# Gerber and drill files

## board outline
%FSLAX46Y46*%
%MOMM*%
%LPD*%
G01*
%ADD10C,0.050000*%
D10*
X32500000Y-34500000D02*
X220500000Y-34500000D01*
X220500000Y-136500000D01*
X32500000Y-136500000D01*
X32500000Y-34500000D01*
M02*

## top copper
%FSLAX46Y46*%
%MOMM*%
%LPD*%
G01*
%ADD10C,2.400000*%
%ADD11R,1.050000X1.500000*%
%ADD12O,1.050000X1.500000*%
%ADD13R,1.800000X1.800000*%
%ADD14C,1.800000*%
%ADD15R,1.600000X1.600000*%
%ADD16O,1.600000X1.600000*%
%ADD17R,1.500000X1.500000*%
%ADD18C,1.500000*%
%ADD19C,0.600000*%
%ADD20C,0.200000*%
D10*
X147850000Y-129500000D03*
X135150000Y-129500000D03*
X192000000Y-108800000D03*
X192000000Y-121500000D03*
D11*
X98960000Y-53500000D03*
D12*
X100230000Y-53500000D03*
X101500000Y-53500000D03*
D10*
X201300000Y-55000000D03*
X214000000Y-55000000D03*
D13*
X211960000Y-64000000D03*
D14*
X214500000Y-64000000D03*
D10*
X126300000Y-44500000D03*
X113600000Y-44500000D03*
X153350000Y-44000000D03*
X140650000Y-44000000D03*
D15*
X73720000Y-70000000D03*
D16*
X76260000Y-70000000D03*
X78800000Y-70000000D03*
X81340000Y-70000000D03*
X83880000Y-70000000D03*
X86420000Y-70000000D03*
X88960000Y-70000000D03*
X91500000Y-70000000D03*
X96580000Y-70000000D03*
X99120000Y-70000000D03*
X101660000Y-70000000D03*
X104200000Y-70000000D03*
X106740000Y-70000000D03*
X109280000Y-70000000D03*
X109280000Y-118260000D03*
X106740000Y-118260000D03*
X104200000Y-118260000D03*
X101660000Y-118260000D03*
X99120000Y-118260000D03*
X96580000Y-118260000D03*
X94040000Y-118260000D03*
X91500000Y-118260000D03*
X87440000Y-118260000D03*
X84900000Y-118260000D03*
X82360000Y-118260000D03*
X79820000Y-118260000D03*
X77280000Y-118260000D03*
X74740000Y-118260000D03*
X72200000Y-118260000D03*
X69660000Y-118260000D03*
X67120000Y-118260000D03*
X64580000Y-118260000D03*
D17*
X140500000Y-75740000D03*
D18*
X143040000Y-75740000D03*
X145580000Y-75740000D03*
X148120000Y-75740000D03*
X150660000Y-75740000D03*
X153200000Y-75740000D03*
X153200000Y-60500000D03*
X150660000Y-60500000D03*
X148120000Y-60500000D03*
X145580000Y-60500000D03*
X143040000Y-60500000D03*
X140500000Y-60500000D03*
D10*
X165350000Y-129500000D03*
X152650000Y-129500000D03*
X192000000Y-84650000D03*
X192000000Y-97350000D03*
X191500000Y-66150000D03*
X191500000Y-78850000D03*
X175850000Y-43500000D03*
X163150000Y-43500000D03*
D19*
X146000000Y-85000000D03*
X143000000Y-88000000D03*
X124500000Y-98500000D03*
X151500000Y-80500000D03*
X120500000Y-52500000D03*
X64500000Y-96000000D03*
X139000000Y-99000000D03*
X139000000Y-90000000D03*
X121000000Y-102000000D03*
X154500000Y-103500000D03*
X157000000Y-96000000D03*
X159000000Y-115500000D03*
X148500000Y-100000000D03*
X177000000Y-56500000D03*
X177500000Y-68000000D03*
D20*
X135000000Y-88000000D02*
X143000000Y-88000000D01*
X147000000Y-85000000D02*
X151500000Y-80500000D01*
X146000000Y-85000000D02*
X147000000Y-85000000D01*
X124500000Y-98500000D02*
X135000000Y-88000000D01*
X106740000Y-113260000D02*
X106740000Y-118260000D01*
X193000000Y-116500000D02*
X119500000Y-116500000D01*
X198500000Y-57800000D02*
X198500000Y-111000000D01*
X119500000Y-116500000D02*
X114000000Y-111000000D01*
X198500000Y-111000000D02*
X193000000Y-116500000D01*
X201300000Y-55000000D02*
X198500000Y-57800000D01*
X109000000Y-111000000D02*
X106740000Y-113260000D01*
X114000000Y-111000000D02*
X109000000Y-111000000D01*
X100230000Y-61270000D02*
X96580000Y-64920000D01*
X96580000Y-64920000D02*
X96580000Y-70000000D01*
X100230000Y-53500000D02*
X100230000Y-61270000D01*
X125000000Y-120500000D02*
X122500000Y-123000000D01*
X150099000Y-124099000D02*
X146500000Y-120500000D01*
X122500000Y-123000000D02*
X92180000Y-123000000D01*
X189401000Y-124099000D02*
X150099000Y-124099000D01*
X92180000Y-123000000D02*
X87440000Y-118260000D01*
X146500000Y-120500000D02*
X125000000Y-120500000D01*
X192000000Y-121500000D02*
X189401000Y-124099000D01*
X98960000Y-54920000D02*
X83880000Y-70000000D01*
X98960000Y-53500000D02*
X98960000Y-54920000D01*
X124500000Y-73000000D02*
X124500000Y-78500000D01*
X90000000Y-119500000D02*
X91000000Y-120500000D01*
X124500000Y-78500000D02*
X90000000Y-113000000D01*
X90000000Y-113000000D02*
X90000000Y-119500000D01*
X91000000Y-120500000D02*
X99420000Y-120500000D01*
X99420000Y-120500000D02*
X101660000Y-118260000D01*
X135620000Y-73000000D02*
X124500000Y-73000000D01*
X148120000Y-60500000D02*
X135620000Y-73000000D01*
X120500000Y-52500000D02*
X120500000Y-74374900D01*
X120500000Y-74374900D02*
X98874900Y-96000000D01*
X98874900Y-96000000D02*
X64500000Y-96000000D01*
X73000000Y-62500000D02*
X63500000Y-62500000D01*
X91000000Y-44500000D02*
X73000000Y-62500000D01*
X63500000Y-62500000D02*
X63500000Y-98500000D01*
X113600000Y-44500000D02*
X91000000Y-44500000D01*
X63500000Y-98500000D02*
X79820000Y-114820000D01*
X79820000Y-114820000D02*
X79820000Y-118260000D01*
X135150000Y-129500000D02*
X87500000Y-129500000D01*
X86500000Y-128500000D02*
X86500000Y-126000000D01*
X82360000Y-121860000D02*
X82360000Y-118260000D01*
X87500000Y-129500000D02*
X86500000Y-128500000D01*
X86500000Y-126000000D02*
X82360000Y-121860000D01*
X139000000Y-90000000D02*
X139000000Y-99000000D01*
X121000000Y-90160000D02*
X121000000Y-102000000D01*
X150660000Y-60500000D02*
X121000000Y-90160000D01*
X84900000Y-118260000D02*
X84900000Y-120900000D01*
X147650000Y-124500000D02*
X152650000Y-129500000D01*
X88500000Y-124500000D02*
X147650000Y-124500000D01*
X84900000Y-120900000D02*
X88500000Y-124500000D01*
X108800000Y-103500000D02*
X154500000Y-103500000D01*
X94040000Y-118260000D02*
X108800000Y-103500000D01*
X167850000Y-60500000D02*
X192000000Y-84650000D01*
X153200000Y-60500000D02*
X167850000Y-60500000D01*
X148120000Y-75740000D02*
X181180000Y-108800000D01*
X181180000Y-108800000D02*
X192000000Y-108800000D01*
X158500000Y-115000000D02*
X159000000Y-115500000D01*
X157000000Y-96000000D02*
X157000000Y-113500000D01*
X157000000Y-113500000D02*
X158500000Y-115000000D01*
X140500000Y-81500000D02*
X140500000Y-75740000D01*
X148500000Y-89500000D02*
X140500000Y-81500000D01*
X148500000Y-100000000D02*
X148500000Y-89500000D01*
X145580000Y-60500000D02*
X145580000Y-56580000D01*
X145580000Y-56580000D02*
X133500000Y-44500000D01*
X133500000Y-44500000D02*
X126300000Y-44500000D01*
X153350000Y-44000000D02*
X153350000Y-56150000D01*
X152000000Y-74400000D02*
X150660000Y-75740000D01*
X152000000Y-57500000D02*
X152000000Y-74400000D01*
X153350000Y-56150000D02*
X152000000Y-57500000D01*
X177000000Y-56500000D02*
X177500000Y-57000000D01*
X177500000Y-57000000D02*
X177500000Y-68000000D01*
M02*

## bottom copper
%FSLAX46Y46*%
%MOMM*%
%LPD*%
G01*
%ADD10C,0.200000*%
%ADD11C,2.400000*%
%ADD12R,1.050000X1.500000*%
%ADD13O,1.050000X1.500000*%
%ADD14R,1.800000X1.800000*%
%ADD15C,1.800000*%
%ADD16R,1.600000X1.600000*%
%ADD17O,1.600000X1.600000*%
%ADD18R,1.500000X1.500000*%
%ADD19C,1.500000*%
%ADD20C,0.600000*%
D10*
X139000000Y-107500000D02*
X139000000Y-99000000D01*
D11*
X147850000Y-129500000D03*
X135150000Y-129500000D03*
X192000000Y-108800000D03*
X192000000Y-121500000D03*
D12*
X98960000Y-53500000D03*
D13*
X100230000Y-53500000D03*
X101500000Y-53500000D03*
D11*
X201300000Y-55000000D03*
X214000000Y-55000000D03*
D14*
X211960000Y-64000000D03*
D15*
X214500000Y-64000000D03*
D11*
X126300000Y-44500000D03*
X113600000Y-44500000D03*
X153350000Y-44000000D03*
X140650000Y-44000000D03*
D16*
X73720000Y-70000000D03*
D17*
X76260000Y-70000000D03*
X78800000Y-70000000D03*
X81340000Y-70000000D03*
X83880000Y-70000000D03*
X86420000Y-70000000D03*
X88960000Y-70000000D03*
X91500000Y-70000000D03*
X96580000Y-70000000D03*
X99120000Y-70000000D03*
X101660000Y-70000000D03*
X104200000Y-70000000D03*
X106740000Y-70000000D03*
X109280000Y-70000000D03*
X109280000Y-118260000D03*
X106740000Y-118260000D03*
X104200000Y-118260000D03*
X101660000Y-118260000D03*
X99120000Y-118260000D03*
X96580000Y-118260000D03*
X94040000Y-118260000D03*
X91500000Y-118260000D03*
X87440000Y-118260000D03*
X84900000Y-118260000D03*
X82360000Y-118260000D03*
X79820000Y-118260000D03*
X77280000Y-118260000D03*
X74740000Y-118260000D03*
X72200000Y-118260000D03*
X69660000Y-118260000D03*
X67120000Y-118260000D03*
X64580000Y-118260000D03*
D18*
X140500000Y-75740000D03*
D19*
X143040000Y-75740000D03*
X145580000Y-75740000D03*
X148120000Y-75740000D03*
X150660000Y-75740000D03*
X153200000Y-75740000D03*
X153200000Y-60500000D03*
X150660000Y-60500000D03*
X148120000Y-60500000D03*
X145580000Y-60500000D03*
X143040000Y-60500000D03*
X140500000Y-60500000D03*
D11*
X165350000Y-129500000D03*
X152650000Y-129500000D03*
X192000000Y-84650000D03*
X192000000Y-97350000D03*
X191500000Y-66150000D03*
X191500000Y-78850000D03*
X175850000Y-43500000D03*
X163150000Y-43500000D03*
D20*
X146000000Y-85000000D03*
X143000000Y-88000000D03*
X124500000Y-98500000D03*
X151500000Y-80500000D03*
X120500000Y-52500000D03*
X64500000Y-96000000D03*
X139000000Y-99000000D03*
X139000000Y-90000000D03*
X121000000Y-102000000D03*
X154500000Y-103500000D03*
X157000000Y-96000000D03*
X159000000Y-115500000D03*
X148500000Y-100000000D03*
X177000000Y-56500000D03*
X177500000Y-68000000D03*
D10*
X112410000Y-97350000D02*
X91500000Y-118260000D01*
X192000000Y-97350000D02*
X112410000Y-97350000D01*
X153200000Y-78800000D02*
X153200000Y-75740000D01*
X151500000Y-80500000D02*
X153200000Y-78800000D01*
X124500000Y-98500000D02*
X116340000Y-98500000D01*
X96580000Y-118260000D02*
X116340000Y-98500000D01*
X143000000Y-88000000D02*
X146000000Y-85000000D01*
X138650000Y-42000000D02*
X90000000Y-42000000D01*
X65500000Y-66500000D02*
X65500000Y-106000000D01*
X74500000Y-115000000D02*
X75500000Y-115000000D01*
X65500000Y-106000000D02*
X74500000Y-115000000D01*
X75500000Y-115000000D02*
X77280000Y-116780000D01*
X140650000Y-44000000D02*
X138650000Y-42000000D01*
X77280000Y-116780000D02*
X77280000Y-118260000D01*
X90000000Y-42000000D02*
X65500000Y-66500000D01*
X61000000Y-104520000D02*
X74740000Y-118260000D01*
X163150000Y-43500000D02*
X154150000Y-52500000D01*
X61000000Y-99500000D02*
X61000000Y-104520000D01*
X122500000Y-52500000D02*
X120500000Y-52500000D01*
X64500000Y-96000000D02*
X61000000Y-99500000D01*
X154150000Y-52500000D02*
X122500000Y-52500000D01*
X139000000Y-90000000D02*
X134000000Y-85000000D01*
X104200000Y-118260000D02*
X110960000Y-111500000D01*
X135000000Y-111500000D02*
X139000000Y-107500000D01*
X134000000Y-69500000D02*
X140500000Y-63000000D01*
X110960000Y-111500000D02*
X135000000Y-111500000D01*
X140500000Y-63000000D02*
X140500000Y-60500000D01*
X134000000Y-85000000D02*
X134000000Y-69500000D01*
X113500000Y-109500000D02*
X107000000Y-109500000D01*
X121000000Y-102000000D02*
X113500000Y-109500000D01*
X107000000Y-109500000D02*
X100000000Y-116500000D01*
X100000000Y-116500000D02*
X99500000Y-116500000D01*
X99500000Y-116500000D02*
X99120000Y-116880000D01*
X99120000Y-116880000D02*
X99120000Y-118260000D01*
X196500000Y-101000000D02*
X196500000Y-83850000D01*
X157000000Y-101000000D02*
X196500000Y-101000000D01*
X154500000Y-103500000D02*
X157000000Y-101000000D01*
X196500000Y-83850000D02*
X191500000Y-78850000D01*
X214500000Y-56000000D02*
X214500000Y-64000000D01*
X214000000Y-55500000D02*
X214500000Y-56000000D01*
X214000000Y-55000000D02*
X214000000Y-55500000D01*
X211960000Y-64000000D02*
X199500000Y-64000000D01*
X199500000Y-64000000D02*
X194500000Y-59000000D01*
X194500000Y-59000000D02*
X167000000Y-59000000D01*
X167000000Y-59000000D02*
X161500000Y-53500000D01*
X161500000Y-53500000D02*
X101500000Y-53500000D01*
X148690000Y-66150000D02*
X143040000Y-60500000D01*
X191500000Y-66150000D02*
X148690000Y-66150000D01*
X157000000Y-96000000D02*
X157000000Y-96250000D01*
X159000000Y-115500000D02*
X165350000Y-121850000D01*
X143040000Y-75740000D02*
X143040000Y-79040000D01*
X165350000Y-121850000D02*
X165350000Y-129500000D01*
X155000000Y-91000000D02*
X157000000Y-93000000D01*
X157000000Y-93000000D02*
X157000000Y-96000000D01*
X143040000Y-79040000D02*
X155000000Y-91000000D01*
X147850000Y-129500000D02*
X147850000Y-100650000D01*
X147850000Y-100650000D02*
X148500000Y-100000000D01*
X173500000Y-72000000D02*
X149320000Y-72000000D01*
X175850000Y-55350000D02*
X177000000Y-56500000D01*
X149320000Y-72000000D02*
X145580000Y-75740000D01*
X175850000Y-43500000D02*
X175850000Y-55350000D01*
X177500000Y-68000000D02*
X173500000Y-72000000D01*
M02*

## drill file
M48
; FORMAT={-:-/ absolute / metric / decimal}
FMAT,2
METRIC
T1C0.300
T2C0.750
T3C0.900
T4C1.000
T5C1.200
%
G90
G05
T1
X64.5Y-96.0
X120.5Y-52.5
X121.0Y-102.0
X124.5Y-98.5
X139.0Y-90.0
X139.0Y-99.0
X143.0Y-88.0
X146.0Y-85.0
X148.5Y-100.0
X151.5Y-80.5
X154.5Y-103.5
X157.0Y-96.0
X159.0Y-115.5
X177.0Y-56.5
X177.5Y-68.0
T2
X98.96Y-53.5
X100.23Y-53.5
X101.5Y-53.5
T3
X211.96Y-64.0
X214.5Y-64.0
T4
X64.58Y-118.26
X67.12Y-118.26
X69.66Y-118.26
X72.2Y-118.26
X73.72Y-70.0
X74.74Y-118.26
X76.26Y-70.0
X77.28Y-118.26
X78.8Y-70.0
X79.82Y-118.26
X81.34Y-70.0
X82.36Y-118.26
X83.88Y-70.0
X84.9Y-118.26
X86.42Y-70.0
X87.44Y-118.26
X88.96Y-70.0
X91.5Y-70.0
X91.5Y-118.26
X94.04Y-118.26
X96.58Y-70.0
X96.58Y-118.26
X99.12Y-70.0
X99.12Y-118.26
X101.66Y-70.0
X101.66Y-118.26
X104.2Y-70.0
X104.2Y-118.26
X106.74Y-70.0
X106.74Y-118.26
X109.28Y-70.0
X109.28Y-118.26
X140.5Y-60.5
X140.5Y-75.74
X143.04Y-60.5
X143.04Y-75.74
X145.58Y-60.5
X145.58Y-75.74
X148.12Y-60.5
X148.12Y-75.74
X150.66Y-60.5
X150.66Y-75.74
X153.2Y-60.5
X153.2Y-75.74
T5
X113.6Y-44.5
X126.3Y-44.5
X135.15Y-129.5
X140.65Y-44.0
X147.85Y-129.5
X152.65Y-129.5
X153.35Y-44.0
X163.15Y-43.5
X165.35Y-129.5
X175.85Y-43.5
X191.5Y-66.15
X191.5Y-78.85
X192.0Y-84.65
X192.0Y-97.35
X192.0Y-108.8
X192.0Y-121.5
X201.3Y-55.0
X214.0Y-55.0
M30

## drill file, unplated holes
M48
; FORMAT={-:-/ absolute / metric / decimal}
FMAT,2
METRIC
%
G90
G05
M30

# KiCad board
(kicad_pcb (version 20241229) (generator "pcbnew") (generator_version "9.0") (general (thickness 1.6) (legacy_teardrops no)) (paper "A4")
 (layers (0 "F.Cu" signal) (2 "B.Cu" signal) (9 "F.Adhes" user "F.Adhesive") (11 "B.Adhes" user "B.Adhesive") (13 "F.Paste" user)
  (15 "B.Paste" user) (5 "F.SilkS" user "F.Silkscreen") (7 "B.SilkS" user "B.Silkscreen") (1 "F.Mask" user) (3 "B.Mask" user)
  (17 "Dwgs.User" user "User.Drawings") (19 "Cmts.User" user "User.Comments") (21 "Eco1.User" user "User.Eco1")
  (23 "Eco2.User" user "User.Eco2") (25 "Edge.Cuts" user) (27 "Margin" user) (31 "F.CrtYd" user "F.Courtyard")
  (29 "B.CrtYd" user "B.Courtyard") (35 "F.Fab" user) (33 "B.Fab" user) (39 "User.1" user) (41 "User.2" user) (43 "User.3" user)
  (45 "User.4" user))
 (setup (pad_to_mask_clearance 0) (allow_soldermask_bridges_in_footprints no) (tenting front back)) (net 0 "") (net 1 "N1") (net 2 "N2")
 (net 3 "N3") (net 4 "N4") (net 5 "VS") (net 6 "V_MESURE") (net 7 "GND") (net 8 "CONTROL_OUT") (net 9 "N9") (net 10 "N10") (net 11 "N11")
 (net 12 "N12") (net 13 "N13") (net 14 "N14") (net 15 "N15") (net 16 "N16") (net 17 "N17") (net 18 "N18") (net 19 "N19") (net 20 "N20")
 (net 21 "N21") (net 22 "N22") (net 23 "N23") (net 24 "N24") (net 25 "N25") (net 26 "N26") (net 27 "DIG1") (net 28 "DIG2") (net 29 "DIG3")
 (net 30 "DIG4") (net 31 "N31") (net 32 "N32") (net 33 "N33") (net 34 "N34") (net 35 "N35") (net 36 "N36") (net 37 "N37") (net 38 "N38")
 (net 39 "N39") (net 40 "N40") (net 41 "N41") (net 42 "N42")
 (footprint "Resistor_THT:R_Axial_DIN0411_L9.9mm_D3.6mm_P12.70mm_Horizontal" (layer "F.Cu") (at 147.85 129.5 180)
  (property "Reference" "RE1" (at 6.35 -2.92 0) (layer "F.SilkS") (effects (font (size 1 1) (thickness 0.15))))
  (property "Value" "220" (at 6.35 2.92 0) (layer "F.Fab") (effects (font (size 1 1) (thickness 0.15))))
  (pad "1" thru_hole circle (at 0 0 180) (size 2.4 2.4) (drill 1.2) (layers "*.Cu" "*.Mask") (remove_unused_layers no) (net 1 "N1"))
  (pad "2" thru_hole circle (at 12.7 0 180) (size 2.4 2.4) (drill 1.2) (layers "*.Cu" "*.Mask") (remove_unused_layers no) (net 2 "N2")))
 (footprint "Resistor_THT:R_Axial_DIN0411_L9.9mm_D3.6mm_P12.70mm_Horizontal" (layer "F.Cu") (at 192 108.8 -90)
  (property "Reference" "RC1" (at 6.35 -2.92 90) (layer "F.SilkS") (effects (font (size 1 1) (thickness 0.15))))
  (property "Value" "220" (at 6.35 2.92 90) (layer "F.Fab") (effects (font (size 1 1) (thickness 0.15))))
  (pad "1" thru_hole circle (at 0 0 270) (size 2.4 2.4) (drill 1.2) (layers "*.Cu" "*.Mask") (remove_unused_layers no) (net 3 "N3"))
  (pad "2" thru_hole circle (at 12.7 0 270) (size 2.4 2.4) (drill 1.2) (layers "*.Cu" "*.Mask") (remove_unused_layers no) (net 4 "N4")))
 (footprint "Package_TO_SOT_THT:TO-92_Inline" (layer "F.Cu") (at 98.96 53.5)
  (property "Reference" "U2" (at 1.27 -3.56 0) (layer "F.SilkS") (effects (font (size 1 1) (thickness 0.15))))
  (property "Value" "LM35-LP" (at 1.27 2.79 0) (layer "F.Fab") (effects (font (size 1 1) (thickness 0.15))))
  (pad "1" thru_hole rect (at 0 0) (size 1.05 1.5) (drill 0.75) (layers "*.Cu" "*.Mask") (remove_unused_layers no) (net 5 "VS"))
  (pad "2" thru_hole oval (at 1.27 0) (size 1.05 1.5) (drill 0.75) (layers "*.Cu" "*.Mask") (remove_unused_layers no) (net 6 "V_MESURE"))
  (pad "3" thru_hole oval (at 2.54 0) (size 1.05 1.5) (drill 0.75) (layers "*.Cu" "*.Mask") (remove_unused_layers no) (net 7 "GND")))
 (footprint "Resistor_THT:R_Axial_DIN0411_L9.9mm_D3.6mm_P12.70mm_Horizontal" (layer "F.Cu") (at 201.3 55)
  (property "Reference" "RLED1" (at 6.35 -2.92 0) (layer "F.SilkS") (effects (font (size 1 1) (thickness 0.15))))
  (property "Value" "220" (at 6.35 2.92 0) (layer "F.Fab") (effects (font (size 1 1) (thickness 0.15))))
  (pad "1" thru_hole circle (at 0 0) (size 2.4 2.4) (drill 1.2) (layers "*.Cu" "*.Mask") (remove_unused_layers no) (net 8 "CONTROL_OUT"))
  (pad "2" thru_hole circle (at 12.7 0) (size 2.4 2.4) (drill 1.2) (layers "*.Cu" "*.Mask") (remove_unused_layers no) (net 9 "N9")))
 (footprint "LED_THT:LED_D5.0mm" (layer "F.Cu") (at 211.96 64)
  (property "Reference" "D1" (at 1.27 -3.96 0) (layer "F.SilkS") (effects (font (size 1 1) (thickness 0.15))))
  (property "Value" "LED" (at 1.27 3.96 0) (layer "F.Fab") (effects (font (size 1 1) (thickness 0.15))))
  (pad "1" thru_hole rect (at 0 0) (size 1.8 1.8) (drill 0.9) (layers "*.Cu" "*.Mask") (remove_unused_layers no) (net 7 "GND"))
  (pad "2" thru_hole circle (at 2.54 0) (size 1.8 1.8) (drill 0.9) (layers "*.Cu" "*.Mask") (remove_unused_layers no) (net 9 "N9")))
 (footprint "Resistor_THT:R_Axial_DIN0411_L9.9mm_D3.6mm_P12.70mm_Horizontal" (layer "F.Cu") (at 126.3 44.5 180)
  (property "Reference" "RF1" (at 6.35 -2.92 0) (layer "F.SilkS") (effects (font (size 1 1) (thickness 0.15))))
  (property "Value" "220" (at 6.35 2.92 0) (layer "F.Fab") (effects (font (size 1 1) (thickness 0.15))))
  (pad "1" thru_hole circle (at 0 0 180) (size 2.4 2.4) (drill 1.2) (layers "*.Cu" "*.Mask") (remove_unused_layers no) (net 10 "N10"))
  (pad "2" thru_hole circle (at 12.7 0 180) (size 2.4 2.4) (drill 1.2) (layers "*.Cu" "*.Mask") (remove_unused_layers no) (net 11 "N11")))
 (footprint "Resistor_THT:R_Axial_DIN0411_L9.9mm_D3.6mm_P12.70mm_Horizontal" (layer "F.Cu") (at 153.35 44 180)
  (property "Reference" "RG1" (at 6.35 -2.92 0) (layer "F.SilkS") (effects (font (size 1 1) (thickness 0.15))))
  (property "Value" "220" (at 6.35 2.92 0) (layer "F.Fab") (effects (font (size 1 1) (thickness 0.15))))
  (pad "1" thru_hole circle (at 0 0 180) (size 2.4 2.4) (drill 1.2) (layers "*.Cu" "*.Mask") (remove_unused_layers no) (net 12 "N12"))
  (pad "2" thru_hole circle (at 12.7 0 180) (size 2.4 2.4) (drill 1.2) (layers "*.Cu" "*.Mask") (remove_unused_layers no) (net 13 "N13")))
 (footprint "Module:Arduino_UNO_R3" (layer "F.Cu") (at 73.72 70)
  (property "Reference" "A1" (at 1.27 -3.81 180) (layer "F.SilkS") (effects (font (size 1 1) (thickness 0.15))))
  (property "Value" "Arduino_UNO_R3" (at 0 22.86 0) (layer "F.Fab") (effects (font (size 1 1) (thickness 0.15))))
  (pad "1" thru_hole rect (at 0 0 90) (size 1.6 1.6) (drill 1) (layers "*.Cu" "*.Mask") (remove_unused_layers no) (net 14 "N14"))
  (pad "2" thru_hole oval (at 2.54 0 90) (size 1.6 1.6) (drill 1) (layers "*.Cu" "*.Mask") (remove_unused_layers no) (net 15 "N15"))
  (pad "3" thru_hole oval (at 5.08 0 90) (size 1.6 1.6) (drill 1) (layers "*.Cu" "*.Mask") (remove_unused_layers no) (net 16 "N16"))
  (pad "4" thru_hole oval (at 7.62 0 90) (size 1.6 1.6) (drill 1) (layers "*.Cu" "*.Mask") (remove_unused_layers no) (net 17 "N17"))
  (pad "5" thru_hole oval (at 10.16 0 90) (size 1.6 1.6) (drill 1) (layers "*.Cu" "*.Mask") (remove_unused_layers no) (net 5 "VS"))
  (pad "6" thru_hole oval (at 12.7 0 90) (size 1.6 1.6) (drill 1) (layers "*.Cu" "*.Mask") (remove_unused_layers no) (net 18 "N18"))
  (pad "7" thru_hole oval (at 15.24 0 90) (size 1.6 1.6) (drill 1) (layers "*.Cu" "*.Mask") (remove_unused_layers no) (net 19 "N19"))
  (pad "8" thru_hole oval (at 17.78 0 90) (size 1.6 1.6) (drill 1) (layers "*.Cu" "*.Mask") (remove_unused_layers no) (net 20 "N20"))
  (pad "9" thru_hole oval (at 22.86 0 90) (size 1.6 1.6) (drill 1) (layers "*.Cu" "*.Mask") (remove_unused_layers no) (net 6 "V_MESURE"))
  (pad "10" thru_hole oval (at 25.4 0 90) (size 1.6 1.6) (drill 1) (layers "*.Cu" "*.Mask") (remove_unused_layers no) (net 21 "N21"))
  (pad "11" thru_hole oval (at 27.94 0 90) (size 1.6 1.6) (drill 1) (layers "*.Cu" "*.Mask") (remove_unused_layers no) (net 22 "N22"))
  (pad "12" thru_hole oval (at 30.48 0 90) (size 1.6 1.6) (drill 1) (layers "*.Cu" "*.Mask") (remove_unused_layers no) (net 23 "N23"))
  (pad "13" thru_hole oval (at 33.02 0 90) (size 1.6 1.6) (drill 1) (layers "*.Cu" "*.Mask") (remove_unused_layers no) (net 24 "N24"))
  (pad "14" thru_hole oval (at 35.56 0 90) (size 1.6 1.6) (drill 1) (layers "*.Cu" "*.Mask") (remove_unused_layers no) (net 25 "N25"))
  (pad "15" thru_hole oval (at 35.56 48.26 90) (size 1.6 1.6) (drill 1) (layers "*.Cu" "*.Mask") (remove_unused_layers no) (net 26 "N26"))
  (pad "16" thru_hole oval (at 33.02 48.26 90) (size 1.6 1.6) (drill 1) (layers "*.Cu" "*.Mask") (remove_unused_layers no)
   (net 8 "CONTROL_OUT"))
  (pad "17" thru_hole oval (at 30.48 48.26 90) (size 1.6 1.6) (drill 1) (layers "*.Cu" "*.Mask") (remove_unused_layers no) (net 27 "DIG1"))
  (pad "18" thru_hole oval (at 27.94 48.26 90) (size 1.6 1.6) (drill 1) (layers "*.Cu" "*.Mask") (remove_unused_layers no) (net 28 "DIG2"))
  (pad "19" thru_hole oval (at 25.4 48.26 90) (size 1.6 1.6) (drill 1) (layers "*.Cu" "*.Mask") (remove_unused_layers no) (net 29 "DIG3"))
  (pad "20" thru_hole oval (at 22.86 48.26 90) (size 1.6 1.6) (drill 1) (layers "*.Cu" "*.Mask") (remove_unused_layers no) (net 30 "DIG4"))
  (pad "21" thru_hole oval (at 20.32 48.26 90) (size 1.6 1.6) (drill 1) (layers "*.Cu" "*.Mask") (remove_unused_layers no) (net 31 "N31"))
  (pad "22" thru_hole oval (at 17.78 48.26 90) (size 1.6 1.6) (drill 1) (layers "*.Cu" "*.Mask") (remove_unused_layers no) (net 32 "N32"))
  (pad "23" thru_hole oval (at 13.72 48.26 90) (size 1.6 1.6) (drill 1) (layers "*.Cu" "*.Mask") (remove_unused_layers no) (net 4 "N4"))
  (pad "24" thru_hole oval (at 11.18 48.26 90) (size 1.6 1.6) (drill 1) (layers "*.Cu" "*.Mask") (remove_unused_layers no) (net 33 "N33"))
  (pad "25" thru_hole oval (at 8.64 48.26 90) (size 1.6 1.6) (drill 1) (layers "*.Cu" "*.Mask") (remove_unused_layers no) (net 2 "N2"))
  (pad "26" thru_hole oval (at 6.1 48.26 90) (size 1.6 1.6) (drill 1) (layers "*.Cu" "*.Mask") (remove_unused_layers no) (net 11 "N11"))
  (pad "27" thru_hole oval (at 3.56 48.26 90) (size 1.6 1.6) (drill 1) (layers "*.Cu" "*.Mask") (remove_unused_layers no) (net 13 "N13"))
  (pad "28" thru_hole oval (at 1.02 48.26 90) (size 1.6 1.6) (drill 1) (layers "*.Cu" "*.Mask") (remove_unused_layers no) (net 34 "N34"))
  (pad "29" thru_hole oval (at -1.52 48.26 90) (size 1.6 1.6) (drill 1) (layers "*.Cu" "*.Mask") (remove_unused_layers no) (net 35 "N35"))
  (pad "30" thru_hole oval (at -4.06 48.26 90) (size 1.6 1.6) (drill 1) (layers "*.Cu" "*.Mask") (remove_unused_layers no) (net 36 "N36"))
  (pad "31" thru_hole oval (at -6.6 48.26 90) (size 1.6 1.6) (drill 1) (layers "*.Cu" "*.Mask") (remove_unused_layers no) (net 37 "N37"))
  (pad "32" thru_hole oval (at -9.14 48.26 90) (size 1.6 1.6) (drill 1) (layers "*.Cu" "*.Mask") (remove_unused_layers no) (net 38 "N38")))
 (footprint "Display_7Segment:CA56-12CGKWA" (layer "F.Cu") (at 140.5 75.74 90)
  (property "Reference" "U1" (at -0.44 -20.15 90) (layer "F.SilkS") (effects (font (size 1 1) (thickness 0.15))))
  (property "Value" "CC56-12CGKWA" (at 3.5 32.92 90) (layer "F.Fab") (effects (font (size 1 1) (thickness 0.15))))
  (pad "1" thru_hole rect (at 0 0 90) (size 1.5 1.5) (drill 1) (layers "*.Cu" "*.Mask") (remove_unused_layers no) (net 1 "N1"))
  (pad "2" thru_hole circle (at 0 2.54 90) (size 1.5 1.5) (drill 1) (layers "*.Cu" "*.Mask") (remove_unused_layers no) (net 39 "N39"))
  (pad "3" thru_hole circle (at 0 5.08 90) (size 1.5 1.5) (drill 1) (layers "*.Cu" "*.Mask") (remove_unused_layers no) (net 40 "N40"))
  (pad "4" thru_hole circle (at 0 7.62 90) (size 1.5 1.5) (drill 1) (layers "*.Cu" "*.Mask") (remove_unused_layers no) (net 3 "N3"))
  (pad "5" thru_hole circle (at 0 10.16 90) (size 1.5 1.5) (drill 1) (layers "*.Cu" "*.Mask") (remove_unused_layers no) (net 12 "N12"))
  (pad "6" thru_hole circle (at 0 12.7 90) (size 1.5 1.5) (drill 1) (layers "*.Cu" "*.Mask") (remove_unused_layers no) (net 30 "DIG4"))
  (pad "7" thru_hole circle (at 15.24 12.7 90) (size 1.5 1.5) (drill 1) (layers "*.Cu" "*.Mask") (remove_unused_layers no) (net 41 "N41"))
  (pad "8" thru_hole circle (at 15.24 10.16 90) (size 1.5 1.5) (drill 1) (layers "*.Cu" "*.Mask") (remove_unused_layers no) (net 29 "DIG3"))
  (pad "9" thru_hole circle (at 15.24 7.62 90) (size 1.5 1.5) (drill 1) (layers "*.Cu" "*.Mask") (remove_unused_layers no) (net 28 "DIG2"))
  (pad "10" thru_hole circle (at 15.24 5.08 90) (size 1.5 1.5) (drill 1) (layers "*.Cu" "*.Mask") (remove_unused_layers no) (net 10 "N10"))
  (pad "11" thru_hole circle (at 15.24 2.54 90) (size 1.5 1.5) (drill 1) (layers "*.Cu" "*.Mask") (remove_unused_layers no) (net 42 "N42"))
  (pad "12" thru_hole circle (at 15.24 0 90) (size 1.5 1.5) (drill 1) (layers "*.Cu" "*.Mask") (remove_unused_layers no) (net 27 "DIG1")))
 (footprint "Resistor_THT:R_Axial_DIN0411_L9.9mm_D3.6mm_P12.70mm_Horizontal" (layer "F.Cu") (at 165.35 129.5 180)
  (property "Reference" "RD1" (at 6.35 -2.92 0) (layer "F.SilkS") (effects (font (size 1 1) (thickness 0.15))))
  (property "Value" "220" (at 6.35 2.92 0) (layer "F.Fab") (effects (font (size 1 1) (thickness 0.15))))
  (pad "1" thru_hole circle (at 0 0 180) (size 2.4 2.4) (drill 1.2) (layers "*.Cu" "*.Mask") (remove_unused_layers no) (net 39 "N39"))
  (pad "2" thru_hole circle (at 12.7 0 180) (size 2.4 2.4) (drill 1.2) (layers "*.Cu" "*.Mask") (remove_unused_layers no) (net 33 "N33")))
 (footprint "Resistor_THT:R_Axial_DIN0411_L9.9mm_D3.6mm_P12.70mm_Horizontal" (layer "F.Cu") (at 192 84.65 -90)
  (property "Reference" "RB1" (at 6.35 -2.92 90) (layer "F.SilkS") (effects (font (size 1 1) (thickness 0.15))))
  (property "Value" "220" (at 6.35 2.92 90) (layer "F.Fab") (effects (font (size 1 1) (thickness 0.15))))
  (pad "1" thru_hole circle (at 0 0 270) (size 2.4 2.4) (drill 1.2) (layers "*.Cu" "*.Mask") (remove_unused_layers no) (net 41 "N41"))
  (pad "2" thru_hole circle (at 12.7 0 270) (size 2.4 2.4) (drill 1.2) (layers "*.Cu" "*.Mask") (remove_unused_layers no) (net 32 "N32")))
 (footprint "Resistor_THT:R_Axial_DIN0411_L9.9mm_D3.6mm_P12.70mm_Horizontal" (layer "F.Cu") (at 191.5 66.15 -90)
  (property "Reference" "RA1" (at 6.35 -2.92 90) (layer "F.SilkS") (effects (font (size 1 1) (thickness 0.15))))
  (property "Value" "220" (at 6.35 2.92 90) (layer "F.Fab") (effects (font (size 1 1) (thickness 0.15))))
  (pad "1" thru_hole circle (at 0 0 270) (size 2.4 2.4) (drill 1.2) (layers "*.Cu" "*.Mask") (remove_unused_layers no) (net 42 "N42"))
  (pad "2" thru_hole circle (at 12.7 0 270) (size 2.4 2.4) (drill 1.2) (layers "*.Cu" "*.Mask") (remove_unused_layers no) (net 31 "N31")))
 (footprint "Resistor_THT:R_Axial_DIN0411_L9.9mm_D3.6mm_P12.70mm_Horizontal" (layer "F.Cu") (at 175.85 43.5 180)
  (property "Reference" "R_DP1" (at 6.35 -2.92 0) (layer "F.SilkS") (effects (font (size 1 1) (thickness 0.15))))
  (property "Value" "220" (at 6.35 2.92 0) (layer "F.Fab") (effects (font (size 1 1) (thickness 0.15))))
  (pad "1" thru_hole circle (at 0 0 180) (size 2.4 2.4) (drill 1.2) (layers "*.Cu" "*.Mask") (remove_unused_layers no) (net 40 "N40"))
  (pad "2" thru_hole circle (at 12.7 0 180) (size 2.4 2.4) (drill 1.2) (layers "*.Cu" "*.Mask") (remove_unused_layers no) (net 34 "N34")))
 (gr_line (start 139 107.5) (end 139 99) (stroke (width 0.2) (type default)) (layer "B.Cu") (net 27))
 (gr_rect (start 32.5 34.5) (end 220.5 136.5) (stroke (width 0.05) (type default)) (fill no) (layer "Edge.Cuts"))
 (segment (start 112.41 97.35) (end 91.5 118.26) (width 0.2) (layer "B.Cu") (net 32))
 (segment (start 192 97.35) (end 112.41 97.35) (width 0.2) (layer "B.Cu") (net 32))
 (segment (start 135 88) (end 143 88) (width 0.2) (layer "F.Cu") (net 30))
 (segment (start 147 85) (end 151.5 80.5) (width 0.2) (layer "F.Cu") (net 30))
 (segment (start 146 85) (end 147 85) (width 0.2) (layer "F.Cu") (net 30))
 (segment (start 124.5 98.5) (end 135 88) (width 0.2) (layer "F.Cu") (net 30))
 (via (at 146 85) (size 0.6) (drill 0.3) (layers "F.Cu" "B.Cu") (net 30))
 (via (at 143 88) (size 0.6) (drill 0.3) (layers "F.Cu" "B.Cu") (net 30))
 (via (at 124.5 98.5) (size 0.6) (drill 0.3) (layers "F.Cu" "B.Cu") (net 30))
 (via (at 151.5 80.5) (size 0.6) (drill 0.3) (layers "F.Cu" "B.Cu") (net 30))
 (segment (start 153.2 78.8) (end 153.2 75.74) (width 0.2) (layer "B.Cu") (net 30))
 (segment (start 151.5 80.5) (end 153.2 78.8) (width 0.2) (layer "B.Cu") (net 30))
 (segment (start 124.5 98.5) (end 116.34 98.5) (width 0.2) (layer "B.Cu") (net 30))
 (segment (start 96.58 118.26) (end 116.34 98.5) (width 0.2) (layer "B.Cu") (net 30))
 (segment (start 143 88) (end 146 85) (width 0.2) (layer "B.Cu") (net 30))
 (segment (start 106.74 113.26) (end 106.74 118.26) (width 0.2) (layer "F.Cu") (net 8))
 (segment (start 193 116.5) (end 119.5 116.5) (width 0.2) (layer "F.Cu") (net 8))
 (segment (start 198.5 57.8) (end 198.5 111) (width 0.2) (layer "F.Cu") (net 8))
 (segment (start 119.5 116.5) (end 114 111) (width 0.2) (layer "F.Cu") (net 8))
 (segment (start 198.5 111) (end 193 116.5) (width 0.2) (layer "F.Cu") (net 8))
 (segment (start 201.3 55) (end 198.5 57.8) (width 0.2) (layer "F.Cu") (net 8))
 (segment (start 109 111) (end 106.74 113.26) (width 0.2) (layer "F.Cu") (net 8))
 (segment (start 114 111) (end 109 111) (width 0.2) (layer "F.Cu") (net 8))
 (segment (start 138.65 42) (end 90 42) (width 0.2) (layer "B.Cu") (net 13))
 (segment (start 65.5 66.5) (end 65.5 106) (width 0.2) (layer "B.Cu") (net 13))
 (segment (start 74.5 115) (end 75.5 115) (width 0.2) (layer "B.Cu") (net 13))
 (segment (start 65.5 106) (end 74.5 115) (width 0.2) (layer "B.Cu") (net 13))
 (segment (start 75.5 115) (end 77.28 116.78) (width 0.2) (layer "B.Cu") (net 13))
 (segment (start 140.65 44) (end 138.65 42) (width 0.2) (layer "B.Cu") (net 13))
 (segment (start 77.28 116.78) (end 77.28 118.26) (width 0.2) (layer "B.Cu") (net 13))
 (segment (start 90 42) (end 65.5 66.5) (width 0.2) (layer "B.Cu") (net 13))
 (segment (start 100.23 61.27) (end 96.58 64.92) (width 0.2) (layer "F.Cu") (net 6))
 (segment (start 96.58 64.92) (end 96.58 70) (width 0.2) (layer "F.Cu") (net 6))
 (segment (start 100.23 53.5) (end 100.23 61.27) (width 0.2) (layer "F.Cu") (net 6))
 (segment (start 125 120.5) (end 122.5 123) (width 0.2) (layer "F.Cu") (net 4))
 (segment (start 150.099 124.099) (end 146.5 120.5) (width 0.2) (layer "F.Cu") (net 4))
 (segment (start 122.5 123) (end 92.18 123) (width 0.2) (layer "F.Cu") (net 4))
 (segment (start 189.401 124.099) (end 150.099 124.099) (width 0.2) (layer "F.Cu") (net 4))
 (segment (start 92.18 123) (end 87.44 118.26) (width 0.2) (layer "F.Cu") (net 4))
 (segment (start 146.5 120.5) (end 125 120.5) (width 0.2) (layer "F.Cu") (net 4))
 (segment (start 192 121.5) (end 189.401 124.099) (width 0.2) (layer "F.Cu") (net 4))
 (segment (start 98.96 54.92) (end 83.88 70) (width 0.2) (layer "F.Cu") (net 5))
 (segment (start 98.96 53.5) (end 98.96 54.92) (width 0.2) (layer "F.Cu") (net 5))
 (segment (start 124.5 73) (end 124.5 78.5) (width 0.2) (layer "F.Cu") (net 28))
 (segment (start 90 119.5) (end 91 120.5) (width 0.2) (layer "F.Cu") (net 28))
 (segment (start 124.5 78.5) (end 90 113) (width 0.2) (layer "F.Cu") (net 28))
 (segment (start 90 113) (end 90 119.5) (width 0.2) (layer "F.Cu") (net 28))
 (segment (start 91 120.5) (end 99.42 120.5) (width 0.2) (layer "F.Cu") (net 28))
 (segment (start 99.42 120.5) (end 101.66 118.26) (width 0.2) (layer "F.Cu") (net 28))
 (segment (start 135.62 73) (end 124.5 73) (width 0.2) (layer "F.Cu") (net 28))
 (segment (start 148.12 60.5) (end 135.62 73) (width 0.2) (layer "F.Cu") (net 28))
 (segment (start 120.5 52.5) (end 120.5 74.3749) (width 0.2) (layer "F.Cu") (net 34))
 (segment (start 120.5 74.3749) (end 98.8749 96) (width 0.2) (layer "F.Cu") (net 34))
 (segment (start 98.8749 96) (end 64.5 96) (width 0.2) (layer "F.Cu") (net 34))
 (via (at 120.5 52.5) (size 0.6) (drill 0.3) (layers "F.Cu" "B.Cu") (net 34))
 (via (at 64.5 96) (size 0.6) (drill 0.3) (layers "F.Cu" "B.Cu") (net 34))
 (segment (start 61 104.52) (end 74.74 118.26) (width 0.2) (layer "B.Cu") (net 34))
 (segment (start 163.15 43.5) (end 154.15 52.5) (width 0.2) (layer "B.Cu") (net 34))
 (segment (start 61 99.5) (end 61 104.52) (width 0.2) (layer "B.Cu") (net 34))
 (segment (start 122.5 52.5) (end 120.5 52.5) (width 0.2) (layer "B.Cu") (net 34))
 (segment (start 64.5 96) (end 61 99.5) (width 0.2) (layer "B.Cu") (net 34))
 (segment (start 154.15 52.5) (end 122.5 52.5) (width 0.2) (layer "B.Cu") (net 34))
 (segment (start 73 62.5) (end 63.5 62.5) (width 0.2) (layer "F.Cu") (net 11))
 (segment (start 91 44.5) (end 73 62.5) (width 0.2) (layer "F.Cu") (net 11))
 (segment (start 63.5 62.5) (end 63.5 98.5) (width 0.2) (layer "F.Cu") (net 11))
 (segment (start 113.6 44.5) (end 91 44.5) (width 0.2) (layer "F.Cu") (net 11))
 (segment (start 63.5 98.5) (end 79.82 114.82) (width 0.2) (layer "F.Cu") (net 11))
 (segment (start 79.82 114.82) (end 79.82 118.26) (width 0.2) (layer "F.Cu") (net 11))
 (segment (start 135.15 129.5) (end 87.5 129.5) (width 0.2) (layer "F.Cu") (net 2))
 (segment (start 86.5 128.5) (end 86.5 126) (width 0.2) (layer "F.Cu") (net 2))
 (segment (start 82.36 121.86) (end 82.36 118.26) (width 0.2) (layer "F.Cu") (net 2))
 (segment (start 87.5 129.5) (end 86.5 128.5) (width 0.2) (layer "F.Cu") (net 2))
 (segment (start 86.5 126) (end 82.36 121.86) (width 0.2) (layer "F.Cu") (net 2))
 (segment (start 139 90) (end 139 99) (width 0.2) (layer "F.Cu") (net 27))
 (via (at 139 99) (size 0.6) (drill 0.3) (layers "F.Cu" "B.Cu") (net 27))
 (via (at 139 90) (size 0.6) (drill 0.3) (layers "F.Cu" "B.Cu") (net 27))
 (segment (start 139 90) (end 134 85) (width 0.2) (layer "B.Cu") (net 27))
 (segment (start 104.2 118.26) (end 110.96 111.5) (width 0.2) (layer "B.Cu") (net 27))
 (segment (start 135 111.5) (end 139 107.5) (width 0.2) (layer "B.Cu") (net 27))
 (segment (start 134 69.5) (end 140.5 63) (width 0.2) (layer "B.Cu") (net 27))
 (segment (start 110.96 111.5) (end 135 111.5) (width 0.2) (layer "B.Cu") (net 27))
 (segment (start 140.5 63) (end 140.5 60.5) (width 0.2) (layer "B.Cu") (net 27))
 (segment (start 134 85) (end 134 69.5) (width 0.2) (layer "B.Cu") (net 27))
 (segment (start 121 90.16) (end 121 102) (width 0.2) (layer "F.Cu") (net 29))
 (segment (start 150.66 60.5) (end 121 90.16) (width 0.2) (layer "F.Cu") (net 29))
 (via (at 121 102) (size 0.6) (drill 0.3) (layers "F.Cu" "B.Cu") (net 29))
 (segment (start 113.5 109.5) (end 107 109.5) (width 0.2) (layer "B.Cu") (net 29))
 (segment (start 121 102) (end 113.5 109.5) (width 0.2) (layer "B.Cu") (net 29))
 (segment (start 107 109.5) (end 100 116.5) (width 0.2) (layer "B.Cu") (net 29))
 (segment (start 100 116.5) (end 99.5 116.5) (width 0.2) (layer "B.Cu") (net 29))
 (segment (start 99.5 116.5) (end 99.12 116.88) (width 0.2) (layer "B.Cu") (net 29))
 (segment (start 99.12 116.88) (end 99.12 118.26) (width 0.2) (layer "B.Cu") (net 29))
 (segment (start 84.9 118.26) (end 84.9 120.9) (width 0.2) (layer "F.Cu") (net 33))
 (segment (start 147.65 124.5) (end 152.65 129.5) (width 0.2) (layer "F.Cu") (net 33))
 (segment (start 88.5 124.5) (end 147.65 124.5) (width 0.2) (layer "F.Cu") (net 33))
 (segment (start 84.9 120.9) (end 88.5 124.5) (width 0.2) (layer "F.Cu") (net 33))
 (segment (start 108.8 103.5) (end 154.5 103.5) (width 0.2) (layer "F.Cu") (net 31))
 (segment (start 94.04 118.26) (end 108.8 103.5) (width 0.2) (layer "F.Cu") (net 31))
 (via (at 154.5 103.5) (size 0.6) (drill 0.3) (layers "F.Cu" "B.Cu") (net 31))
 (segment (start 196.5 101) (end 196.5 83.85) (width 0.2) (layer "B.Cu") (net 31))
 (segment (start 157 101) (end 196.5 101) (width 0.2) (layer "B.Cu") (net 31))
 (segment (start 154.5 103.5) (end 157 101) (width 0.2) (layer "B.Cu") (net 31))
 (segment (start 196.5 83.85) (end 191.5 78.85) (width 0.2) (layer "B.Cu") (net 31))
 (segment (start 214.5 56) (end 214.5 64) (width 0.2) (layer "B.Cu") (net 9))
 (segment (start 214 55.5) (end 214.5 56) (width 0.2) (layer "B.Cu") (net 9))
 (segment (start 214 55) (end 214 55.5) (width 0.2) (layer "B.Cu") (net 9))
 (segment (start 211.96 64) (end 199.5 64) (width 0.2) (layer "B.Cu") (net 7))
 (segment (start 199.5 64) (end 194.5 59) (width 0.2) (layer "B.Cu") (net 7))
 (segment (start 194.5 59) (end 167 59) (width 0.2) (layer "B.Cu") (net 7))
 (segment (start 167 59) (end 161.5 53.5) (width 0.2) (layer "B.Cu") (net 7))
 (segment (start 161.5 53.5) (end 101.5 53.5) (width 0.2) (layer "B.Cu") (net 7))
 (segment (start 148.69 66.15) (end 143.04 60.5) (width 0.2) (layer "B.Cu") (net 42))
 (segment (start 191.5 66.15) (end 148.69 66.15) (width 0.2) (layer "B.Cu") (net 42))
 (segment (start 167.85 60.5) (end 192 84.65) (width 0.2) (layer "F.Cu") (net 41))
 (segment (start 153.2 60.5) (end 167.85 60.5) (width 0.2) (layer "F.Cu") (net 41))
 (segment (start 148.12 75.74) (end 181.18 108.8) (width 0.2) (layer "F.Cu") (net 3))
 (segment (start 181.18 108.8) (end 192 108.8) (width 0.2) (layer "F.Cu") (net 3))
 (segment (start 158.5 115) (end 159 115.5) (width 0.2) (layer "F.Cu") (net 39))
 (segment (start 157 96) (end 157 113.5) (width 0.2) (layer "F.Cu") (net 39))
 (segment (start 157 113.5) (end 158.5 115) (width 0.2) (layer "F.Cu") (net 39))
 (via (at 157 96) (size 0.6) (drill 0.3) (layers "F.Cu" "B.Cu") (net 39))
 (via (at 159 115.5) (size 0.6) (drill 0.3) (layers "F.Cu" "B.Cu") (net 39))
 (segment (start 157 96) (end 157 96.25) (width 0.2) (layer "B.Cu") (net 39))
 (segment (start 159 115.5) (end 165.35 121.85) (width 0.2) (layer "B.Cu") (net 39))
 (segment (start 143.04 75.74) (end 143.04 79.04) (width 0.2) (layer "B.Cu") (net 39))
 (segment (start 165.35 121.85) (end 165.35 129.5) (width 0.2) (layer "B.Cu") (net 39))
 (segment (start 155 91) (end 157 93) (width 0.2) (layer "B.Cu") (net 39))
 (segment (start 157 93) (end 157 96) (width 0.2) (layer "B.Cu") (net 39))
 (segment (start 143.04 79.04) (end 155 91) (width 0.2) (layer "B.Cu") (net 39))
 (segment (start 140.5 81.5) (end 140.5 75.74) (width 0.2) (layer "F.Cu") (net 1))
 (segment (start 148.5 89.5) (end 140.5 81.5) (width 0.2) (layer "F.Cu") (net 1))
 (segment (start 148.5 100) (end 148.5 89.5) (width 0.2) (layer "F.Cu") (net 1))
 (via (at 148.5 100) (size 0.6) (drill 0.3) (layers "F.Cu" "B.Cu") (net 1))
 (segment (start 147.85 129.5) (end 147.85 100.65) (width 0.2) (layer "B.Cu") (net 1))
 (segment (start 147.85 100.65) (end 148.5 100) (width 0.2) (layer "B.Cu") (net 1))
 (segment (start 145.58 60.5) (end 145.58 56.58) (width 0.2) (layer "F.Cu") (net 10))
 (segment (start 145.58 56.58) (end 133.5 44.5) (width 0.2) (layer "F.Cu") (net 10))
 (segment (start 133.5 44.5) (end 126.3 44.5) (width 0.2) (layer "F.Cu") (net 10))
 (segment (start 153.35 44) (end 153.35 56.15) (width 0.2) (layer "F.Cu") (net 12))
 (segment (start 152 74.4) (end 150.66 75.74) (width 0.2) (layer "F.Cu") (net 12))
 (segment (start 152 57.5) (end 152 74.4) (width 0.2) (layer "F.Cu") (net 12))
 (segment (start 153.35 56.15) (end 152 57.5) (width 0.2) (layer "F.Cu") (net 12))
 (segment (start 177 56.5) (end 177.5 57) (width 0.2) (layer "F.Cu") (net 40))
 (segment (start 177.5 57) (end 177.5 68) (width 0.2) (layer "F.Cu") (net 40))
 (via (at 177 56.5) (size 0.6) (drill 0.3) (layers "F.Cu" "B.Cu") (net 40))
 (via (at 177.5 68) (size 0.6) (drill 0.3) (layers "F.Cu" "B.Cu") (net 40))
 (segment (start 173.5 72) (end 149.32 72) (width 0.2) (layer "B.Cu") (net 40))
 (segment (start 175.85 55.35) (end 177 56.5) (width 0.2) (layer "B.Cu") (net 40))
 (segment (start 149.32 72) (end 145.58 75.74) (width 0.2) (layer "B.Cu") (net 40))
 (segment (start 175.85 43.5) (end 175.85 55.35) (width 0.2) (layer "B.Cu") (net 40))
 (segment (start 177.5 68) (end 173.5 72) (width 0.2) (layer "B.Cu") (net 40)))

